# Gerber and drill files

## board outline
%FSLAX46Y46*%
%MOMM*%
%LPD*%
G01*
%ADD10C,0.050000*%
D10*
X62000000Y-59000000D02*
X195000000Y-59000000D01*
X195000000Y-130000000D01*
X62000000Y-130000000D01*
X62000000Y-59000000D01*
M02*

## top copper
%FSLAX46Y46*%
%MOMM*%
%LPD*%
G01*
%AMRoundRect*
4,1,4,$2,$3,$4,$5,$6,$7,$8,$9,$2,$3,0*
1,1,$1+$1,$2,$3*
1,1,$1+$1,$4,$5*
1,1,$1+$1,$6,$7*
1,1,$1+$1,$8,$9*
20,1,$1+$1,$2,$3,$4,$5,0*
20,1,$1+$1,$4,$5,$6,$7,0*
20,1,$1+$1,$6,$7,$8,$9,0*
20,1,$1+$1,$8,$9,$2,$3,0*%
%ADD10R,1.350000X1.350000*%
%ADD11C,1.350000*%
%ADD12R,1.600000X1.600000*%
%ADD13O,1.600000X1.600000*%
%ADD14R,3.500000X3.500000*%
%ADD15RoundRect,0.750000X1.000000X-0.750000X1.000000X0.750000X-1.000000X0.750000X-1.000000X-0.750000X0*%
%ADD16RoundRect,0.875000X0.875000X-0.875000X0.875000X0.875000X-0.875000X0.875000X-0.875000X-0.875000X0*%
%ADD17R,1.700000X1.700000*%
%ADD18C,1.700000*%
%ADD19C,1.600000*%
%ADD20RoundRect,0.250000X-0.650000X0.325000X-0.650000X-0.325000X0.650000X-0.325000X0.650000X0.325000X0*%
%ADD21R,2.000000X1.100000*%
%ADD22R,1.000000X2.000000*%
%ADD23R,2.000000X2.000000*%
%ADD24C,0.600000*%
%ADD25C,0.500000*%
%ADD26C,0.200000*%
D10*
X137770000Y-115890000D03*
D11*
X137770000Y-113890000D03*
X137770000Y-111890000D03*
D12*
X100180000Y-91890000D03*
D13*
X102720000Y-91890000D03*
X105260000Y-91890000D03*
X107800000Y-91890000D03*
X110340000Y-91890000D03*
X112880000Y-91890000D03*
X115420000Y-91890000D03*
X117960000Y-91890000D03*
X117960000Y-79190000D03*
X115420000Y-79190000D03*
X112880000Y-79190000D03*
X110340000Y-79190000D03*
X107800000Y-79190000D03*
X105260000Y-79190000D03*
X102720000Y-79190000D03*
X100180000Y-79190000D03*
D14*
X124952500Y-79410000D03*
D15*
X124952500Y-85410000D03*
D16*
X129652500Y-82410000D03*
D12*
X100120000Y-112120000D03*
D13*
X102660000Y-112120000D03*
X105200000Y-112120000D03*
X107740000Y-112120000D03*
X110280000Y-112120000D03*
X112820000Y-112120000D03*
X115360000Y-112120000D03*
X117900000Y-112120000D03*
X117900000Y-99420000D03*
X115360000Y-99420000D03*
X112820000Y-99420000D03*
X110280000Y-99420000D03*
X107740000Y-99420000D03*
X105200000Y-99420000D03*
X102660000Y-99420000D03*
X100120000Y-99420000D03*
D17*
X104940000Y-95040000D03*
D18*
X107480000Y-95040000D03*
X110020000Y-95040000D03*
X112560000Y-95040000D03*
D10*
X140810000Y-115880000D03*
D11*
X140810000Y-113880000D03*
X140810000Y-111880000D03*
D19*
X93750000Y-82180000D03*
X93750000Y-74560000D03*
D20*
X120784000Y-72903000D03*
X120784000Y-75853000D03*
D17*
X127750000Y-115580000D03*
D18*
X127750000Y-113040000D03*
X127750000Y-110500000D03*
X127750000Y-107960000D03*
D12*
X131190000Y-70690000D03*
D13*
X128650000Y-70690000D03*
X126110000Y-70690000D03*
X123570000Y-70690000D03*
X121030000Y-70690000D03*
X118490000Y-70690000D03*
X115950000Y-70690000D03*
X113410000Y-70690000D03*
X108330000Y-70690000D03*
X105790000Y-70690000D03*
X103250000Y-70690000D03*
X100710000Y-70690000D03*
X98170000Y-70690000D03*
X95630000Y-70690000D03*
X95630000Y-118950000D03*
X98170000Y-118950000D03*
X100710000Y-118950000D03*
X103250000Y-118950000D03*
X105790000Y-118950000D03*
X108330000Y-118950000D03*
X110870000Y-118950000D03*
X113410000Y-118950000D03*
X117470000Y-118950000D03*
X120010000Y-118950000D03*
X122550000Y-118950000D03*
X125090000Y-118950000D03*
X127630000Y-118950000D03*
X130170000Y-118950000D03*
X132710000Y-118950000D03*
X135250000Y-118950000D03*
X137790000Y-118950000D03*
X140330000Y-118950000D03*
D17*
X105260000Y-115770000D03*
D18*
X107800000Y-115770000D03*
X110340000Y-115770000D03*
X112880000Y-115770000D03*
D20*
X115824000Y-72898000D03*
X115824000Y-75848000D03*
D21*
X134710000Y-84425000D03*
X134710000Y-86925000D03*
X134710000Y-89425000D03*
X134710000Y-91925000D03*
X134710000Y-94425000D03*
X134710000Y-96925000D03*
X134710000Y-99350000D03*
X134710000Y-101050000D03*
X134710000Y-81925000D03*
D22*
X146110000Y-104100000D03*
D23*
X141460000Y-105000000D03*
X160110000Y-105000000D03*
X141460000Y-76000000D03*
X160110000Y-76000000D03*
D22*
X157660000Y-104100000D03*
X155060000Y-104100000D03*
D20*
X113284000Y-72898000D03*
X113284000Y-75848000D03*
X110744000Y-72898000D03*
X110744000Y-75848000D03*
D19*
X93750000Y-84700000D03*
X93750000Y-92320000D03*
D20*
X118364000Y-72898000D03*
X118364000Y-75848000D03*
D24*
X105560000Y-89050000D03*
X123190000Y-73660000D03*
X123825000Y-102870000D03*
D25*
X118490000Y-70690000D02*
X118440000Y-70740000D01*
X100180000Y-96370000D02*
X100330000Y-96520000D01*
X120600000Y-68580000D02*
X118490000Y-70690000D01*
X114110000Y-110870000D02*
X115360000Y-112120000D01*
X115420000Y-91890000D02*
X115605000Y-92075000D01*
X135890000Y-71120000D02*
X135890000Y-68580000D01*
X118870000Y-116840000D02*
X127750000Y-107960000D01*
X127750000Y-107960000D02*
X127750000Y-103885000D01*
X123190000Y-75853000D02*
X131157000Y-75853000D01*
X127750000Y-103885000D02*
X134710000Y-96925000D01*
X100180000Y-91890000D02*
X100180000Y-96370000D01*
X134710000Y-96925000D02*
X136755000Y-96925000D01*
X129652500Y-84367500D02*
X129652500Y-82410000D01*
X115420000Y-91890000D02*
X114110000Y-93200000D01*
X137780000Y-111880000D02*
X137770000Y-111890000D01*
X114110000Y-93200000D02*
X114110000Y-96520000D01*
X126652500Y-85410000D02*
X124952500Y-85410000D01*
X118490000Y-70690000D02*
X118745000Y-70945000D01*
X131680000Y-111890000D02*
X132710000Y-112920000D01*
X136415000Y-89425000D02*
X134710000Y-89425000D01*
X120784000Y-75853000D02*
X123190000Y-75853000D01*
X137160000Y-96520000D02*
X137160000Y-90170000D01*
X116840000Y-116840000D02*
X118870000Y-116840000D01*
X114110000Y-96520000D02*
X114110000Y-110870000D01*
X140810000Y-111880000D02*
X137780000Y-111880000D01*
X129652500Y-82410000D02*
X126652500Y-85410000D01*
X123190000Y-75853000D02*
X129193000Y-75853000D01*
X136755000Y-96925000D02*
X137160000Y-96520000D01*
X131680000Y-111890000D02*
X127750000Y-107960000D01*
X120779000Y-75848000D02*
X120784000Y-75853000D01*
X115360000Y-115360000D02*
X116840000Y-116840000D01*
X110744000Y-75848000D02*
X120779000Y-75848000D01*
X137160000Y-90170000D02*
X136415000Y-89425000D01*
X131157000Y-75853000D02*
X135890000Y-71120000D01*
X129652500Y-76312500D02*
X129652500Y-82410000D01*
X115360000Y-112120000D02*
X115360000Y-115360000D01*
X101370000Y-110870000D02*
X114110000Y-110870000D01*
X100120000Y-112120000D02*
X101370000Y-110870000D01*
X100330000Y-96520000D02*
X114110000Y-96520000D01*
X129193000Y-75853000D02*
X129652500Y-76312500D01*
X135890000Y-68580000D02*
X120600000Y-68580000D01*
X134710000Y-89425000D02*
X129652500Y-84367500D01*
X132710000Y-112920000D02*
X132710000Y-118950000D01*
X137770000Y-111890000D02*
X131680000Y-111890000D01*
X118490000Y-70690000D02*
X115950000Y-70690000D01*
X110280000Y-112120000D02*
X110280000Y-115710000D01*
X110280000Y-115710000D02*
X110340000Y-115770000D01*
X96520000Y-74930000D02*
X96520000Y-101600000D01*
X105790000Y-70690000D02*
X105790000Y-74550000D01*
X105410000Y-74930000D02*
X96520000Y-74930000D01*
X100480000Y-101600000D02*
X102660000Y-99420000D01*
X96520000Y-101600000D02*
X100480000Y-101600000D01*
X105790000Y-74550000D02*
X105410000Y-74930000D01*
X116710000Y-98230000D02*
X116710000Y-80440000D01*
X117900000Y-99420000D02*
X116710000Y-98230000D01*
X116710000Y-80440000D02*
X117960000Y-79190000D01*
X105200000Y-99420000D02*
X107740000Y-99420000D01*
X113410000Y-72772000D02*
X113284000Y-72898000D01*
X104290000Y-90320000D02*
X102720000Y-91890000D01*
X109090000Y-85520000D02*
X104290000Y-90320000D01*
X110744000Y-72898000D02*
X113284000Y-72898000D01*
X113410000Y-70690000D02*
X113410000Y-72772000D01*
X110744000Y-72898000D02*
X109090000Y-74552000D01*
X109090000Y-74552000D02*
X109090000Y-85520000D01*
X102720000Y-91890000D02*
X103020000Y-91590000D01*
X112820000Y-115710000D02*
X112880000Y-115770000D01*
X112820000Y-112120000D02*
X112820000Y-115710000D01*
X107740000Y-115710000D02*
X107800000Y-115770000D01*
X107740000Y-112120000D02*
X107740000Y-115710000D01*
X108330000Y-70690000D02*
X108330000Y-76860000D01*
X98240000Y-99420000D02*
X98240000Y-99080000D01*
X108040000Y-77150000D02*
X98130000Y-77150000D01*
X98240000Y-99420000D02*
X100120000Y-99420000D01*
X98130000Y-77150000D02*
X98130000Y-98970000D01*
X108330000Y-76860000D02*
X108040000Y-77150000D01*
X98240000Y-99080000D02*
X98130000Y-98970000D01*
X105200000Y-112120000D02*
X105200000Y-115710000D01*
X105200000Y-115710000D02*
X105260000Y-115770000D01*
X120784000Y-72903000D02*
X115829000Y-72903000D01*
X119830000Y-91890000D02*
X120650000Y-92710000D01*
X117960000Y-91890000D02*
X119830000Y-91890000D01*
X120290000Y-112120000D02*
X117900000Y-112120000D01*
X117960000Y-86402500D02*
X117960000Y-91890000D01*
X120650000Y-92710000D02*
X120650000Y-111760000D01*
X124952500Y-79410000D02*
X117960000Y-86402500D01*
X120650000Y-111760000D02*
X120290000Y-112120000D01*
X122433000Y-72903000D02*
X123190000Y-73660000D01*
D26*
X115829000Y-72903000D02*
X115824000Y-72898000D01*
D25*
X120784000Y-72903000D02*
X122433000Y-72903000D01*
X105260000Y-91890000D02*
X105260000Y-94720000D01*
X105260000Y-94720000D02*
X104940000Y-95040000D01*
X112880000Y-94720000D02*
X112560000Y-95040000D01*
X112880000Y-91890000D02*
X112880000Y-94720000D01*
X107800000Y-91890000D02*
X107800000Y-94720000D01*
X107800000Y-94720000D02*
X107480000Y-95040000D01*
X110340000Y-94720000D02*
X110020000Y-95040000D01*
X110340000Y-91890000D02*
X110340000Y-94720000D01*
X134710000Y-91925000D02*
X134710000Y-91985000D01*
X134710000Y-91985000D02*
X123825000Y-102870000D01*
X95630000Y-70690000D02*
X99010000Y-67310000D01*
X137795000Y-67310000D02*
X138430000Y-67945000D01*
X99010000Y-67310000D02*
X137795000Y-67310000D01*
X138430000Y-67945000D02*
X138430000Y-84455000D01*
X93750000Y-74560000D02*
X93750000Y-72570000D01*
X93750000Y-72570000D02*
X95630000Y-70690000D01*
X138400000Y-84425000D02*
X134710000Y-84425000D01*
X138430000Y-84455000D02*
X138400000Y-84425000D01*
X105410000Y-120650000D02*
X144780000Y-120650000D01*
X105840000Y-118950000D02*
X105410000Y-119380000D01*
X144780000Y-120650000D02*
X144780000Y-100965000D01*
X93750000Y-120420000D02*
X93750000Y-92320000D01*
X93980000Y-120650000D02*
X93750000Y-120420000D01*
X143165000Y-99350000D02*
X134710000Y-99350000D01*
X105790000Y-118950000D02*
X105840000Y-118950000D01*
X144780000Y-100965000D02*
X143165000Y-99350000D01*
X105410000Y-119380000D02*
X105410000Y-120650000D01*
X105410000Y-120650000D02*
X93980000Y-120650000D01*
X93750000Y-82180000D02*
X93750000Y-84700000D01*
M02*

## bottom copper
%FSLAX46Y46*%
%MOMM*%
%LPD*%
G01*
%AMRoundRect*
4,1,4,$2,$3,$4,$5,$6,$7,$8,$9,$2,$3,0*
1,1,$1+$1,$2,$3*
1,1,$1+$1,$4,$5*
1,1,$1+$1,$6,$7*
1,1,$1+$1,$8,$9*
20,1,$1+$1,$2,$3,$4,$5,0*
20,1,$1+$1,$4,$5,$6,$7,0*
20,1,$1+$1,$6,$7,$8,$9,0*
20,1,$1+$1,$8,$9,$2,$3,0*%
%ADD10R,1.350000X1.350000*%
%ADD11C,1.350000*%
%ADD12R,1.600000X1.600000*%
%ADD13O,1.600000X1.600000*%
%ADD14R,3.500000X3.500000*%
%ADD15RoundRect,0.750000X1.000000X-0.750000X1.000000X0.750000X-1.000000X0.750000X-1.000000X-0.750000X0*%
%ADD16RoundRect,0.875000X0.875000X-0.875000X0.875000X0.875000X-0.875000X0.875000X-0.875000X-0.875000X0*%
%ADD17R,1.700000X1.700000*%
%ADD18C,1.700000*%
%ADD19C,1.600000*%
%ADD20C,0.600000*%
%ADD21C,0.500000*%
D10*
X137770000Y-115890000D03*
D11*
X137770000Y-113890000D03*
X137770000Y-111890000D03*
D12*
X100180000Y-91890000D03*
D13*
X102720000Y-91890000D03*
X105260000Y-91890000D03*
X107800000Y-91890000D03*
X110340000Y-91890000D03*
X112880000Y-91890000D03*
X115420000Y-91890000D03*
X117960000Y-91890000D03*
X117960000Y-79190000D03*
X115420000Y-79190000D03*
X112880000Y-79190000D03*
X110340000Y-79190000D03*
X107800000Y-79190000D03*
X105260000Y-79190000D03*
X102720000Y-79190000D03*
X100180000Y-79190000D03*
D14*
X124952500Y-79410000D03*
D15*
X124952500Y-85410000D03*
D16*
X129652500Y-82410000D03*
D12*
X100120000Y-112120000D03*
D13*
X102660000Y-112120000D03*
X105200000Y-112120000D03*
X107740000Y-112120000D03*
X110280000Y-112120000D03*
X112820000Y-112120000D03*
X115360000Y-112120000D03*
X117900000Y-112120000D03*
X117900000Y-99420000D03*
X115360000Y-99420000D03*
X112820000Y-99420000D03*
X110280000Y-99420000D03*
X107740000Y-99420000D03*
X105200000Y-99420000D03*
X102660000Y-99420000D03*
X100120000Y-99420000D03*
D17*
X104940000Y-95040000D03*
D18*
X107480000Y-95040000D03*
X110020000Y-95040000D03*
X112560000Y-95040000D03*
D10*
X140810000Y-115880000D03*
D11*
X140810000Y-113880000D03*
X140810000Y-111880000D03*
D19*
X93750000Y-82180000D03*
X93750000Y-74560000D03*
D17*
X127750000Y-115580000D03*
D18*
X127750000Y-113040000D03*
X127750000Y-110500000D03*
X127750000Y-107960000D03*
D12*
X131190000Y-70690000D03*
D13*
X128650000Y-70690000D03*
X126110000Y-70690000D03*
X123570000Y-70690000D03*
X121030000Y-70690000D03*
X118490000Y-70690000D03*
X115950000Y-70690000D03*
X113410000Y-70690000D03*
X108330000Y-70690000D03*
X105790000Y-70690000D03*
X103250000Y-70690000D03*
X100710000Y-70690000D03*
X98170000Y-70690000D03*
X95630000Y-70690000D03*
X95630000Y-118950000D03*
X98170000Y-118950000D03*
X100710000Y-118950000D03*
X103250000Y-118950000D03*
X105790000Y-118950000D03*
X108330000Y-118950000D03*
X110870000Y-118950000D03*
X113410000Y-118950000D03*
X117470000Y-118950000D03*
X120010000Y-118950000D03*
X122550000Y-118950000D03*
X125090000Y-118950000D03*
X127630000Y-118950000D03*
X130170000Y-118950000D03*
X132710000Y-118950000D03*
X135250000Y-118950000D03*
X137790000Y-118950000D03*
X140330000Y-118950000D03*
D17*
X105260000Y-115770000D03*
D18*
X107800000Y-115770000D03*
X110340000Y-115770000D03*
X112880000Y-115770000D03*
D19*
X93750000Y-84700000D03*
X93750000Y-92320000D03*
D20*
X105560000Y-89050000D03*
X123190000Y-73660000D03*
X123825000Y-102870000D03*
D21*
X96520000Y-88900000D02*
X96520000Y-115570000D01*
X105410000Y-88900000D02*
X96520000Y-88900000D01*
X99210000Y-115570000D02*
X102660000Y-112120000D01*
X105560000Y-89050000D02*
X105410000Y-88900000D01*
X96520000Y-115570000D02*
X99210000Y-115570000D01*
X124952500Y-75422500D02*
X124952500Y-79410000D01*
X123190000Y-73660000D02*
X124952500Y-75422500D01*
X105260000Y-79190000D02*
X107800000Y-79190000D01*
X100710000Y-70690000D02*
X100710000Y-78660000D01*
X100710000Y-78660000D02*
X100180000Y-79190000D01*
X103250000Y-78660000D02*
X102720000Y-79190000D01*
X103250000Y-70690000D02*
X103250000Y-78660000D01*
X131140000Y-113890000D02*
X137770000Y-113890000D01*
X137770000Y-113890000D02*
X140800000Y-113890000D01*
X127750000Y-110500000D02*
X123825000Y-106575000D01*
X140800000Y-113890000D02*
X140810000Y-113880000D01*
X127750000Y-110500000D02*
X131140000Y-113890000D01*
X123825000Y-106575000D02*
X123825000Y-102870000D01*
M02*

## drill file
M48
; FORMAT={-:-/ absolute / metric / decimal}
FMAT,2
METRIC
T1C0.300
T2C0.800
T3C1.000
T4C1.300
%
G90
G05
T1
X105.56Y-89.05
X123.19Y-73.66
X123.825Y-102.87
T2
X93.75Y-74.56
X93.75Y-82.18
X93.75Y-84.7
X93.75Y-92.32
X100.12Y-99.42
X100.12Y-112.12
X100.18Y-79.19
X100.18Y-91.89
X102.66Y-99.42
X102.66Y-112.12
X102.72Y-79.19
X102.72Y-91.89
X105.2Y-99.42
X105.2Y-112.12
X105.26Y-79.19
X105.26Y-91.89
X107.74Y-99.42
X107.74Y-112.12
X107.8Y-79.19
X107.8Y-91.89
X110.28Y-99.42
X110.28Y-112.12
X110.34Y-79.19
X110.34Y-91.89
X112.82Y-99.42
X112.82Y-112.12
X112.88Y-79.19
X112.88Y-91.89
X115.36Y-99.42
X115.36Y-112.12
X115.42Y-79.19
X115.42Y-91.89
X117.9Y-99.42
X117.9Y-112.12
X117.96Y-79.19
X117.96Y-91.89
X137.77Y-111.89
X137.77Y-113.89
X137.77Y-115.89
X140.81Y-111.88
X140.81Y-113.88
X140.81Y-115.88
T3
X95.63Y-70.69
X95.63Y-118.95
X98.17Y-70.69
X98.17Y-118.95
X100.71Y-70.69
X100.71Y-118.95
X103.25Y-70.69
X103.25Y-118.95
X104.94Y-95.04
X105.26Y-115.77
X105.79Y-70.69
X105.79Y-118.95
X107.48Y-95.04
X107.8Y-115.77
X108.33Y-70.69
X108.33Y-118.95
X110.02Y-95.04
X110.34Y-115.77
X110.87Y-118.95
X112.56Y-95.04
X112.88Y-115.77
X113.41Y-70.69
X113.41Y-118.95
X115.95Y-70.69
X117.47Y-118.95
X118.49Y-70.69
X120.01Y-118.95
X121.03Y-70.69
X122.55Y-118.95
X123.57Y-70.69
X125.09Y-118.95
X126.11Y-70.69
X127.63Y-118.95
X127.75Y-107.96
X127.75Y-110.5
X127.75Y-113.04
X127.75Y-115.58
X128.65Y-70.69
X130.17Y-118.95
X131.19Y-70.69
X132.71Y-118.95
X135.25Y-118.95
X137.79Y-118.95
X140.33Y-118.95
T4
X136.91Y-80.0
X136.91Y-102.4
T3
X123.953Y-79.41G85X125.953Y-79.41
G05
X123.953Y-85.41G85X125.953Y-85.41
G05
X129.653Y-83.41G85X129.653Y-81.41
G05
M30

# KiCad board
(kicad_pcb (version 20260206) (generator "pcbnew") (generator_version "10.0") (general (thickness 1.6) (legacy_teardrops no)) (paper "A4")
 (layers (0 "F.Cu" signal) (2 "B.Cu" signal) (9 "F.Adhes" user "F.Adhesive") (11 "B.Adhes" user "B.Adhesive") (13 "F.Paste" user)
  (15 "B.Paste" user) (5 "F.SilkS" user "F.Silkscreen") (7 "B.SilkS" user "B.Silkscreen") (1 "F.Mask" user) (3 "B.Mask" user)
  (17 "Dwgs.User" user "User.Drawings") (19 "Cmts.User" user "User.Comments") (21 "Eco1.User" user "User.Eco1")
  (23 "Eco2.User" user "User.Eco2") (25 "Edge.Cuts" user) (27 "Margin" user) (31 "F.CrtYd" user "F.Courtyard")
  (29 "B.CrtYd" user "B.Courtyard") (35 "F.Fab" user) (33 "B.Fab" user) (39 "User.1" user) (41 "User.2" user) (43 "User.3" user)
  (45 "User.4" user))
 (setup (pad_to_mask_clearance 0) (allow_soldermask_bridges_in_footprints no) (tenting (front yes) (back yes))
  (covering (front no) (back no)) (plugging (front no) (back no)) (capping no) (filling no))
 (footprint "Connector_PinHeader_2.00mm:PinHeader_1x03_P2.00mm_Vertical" (layer "F.Cu") (at 137.77 115.89 180)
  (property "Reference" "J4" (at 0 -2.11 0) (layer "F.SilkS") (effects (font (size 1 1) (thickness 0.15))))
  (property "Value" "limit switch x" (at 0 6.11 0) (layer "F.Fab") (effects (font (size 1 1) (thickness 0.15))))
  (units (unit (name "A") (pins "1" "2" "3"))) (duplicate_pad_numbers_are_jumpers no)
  (pad "1" thru_hole rect (at 0 0 180) (size 1.35 1.35) (drill 0.8) (layers "*.Cu" "*.Mask") (remove_unused_layers no) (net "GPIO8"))
  (pad "2" thru_hole circle (at 0 2 180) (size 1.35 1.35) (drill 0.8) (layers "*.Cu" "*.Mask") (remove_unused_layers no) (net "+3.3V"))
  (pad "3" thru_hole circle (at 0 4 180) (size 1.35 1.35) (drill 0.8) (layers "*.Cu" "*.Mask") (remove_unused_layers no) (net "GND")))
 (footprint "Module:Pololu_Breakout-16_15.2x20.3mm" (layer "F.Cu") (at 100.18 91.89 90)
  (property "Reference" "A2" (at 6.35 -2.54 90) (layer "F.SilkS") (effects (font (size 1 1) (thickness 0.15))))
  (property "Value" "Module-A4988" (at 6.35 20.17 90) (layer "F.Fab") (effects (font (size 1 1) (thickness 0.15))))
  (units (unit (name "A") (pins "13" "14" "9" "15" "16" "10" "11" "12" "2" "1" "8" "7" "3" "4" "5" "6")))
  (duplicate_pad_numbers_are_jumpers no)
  (pad "1" thru_hole rect (at 0 0 90) (size 1.6 1.6) (drill 0.8) (layers "*.Cu" "*.Mask") (remove_unused_layers no) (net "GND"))
  (pad "2" thru_hole oval (at 0 2.54 90) (size 1.6 1.6) (drill 0.8) (layers "*.Cu" "*.Mask") (remove_unused_layers no) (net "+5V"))
  (pad "3" thru_hole oval (at 0 5.08 90) (size 1.6 1.6) (drill 0.8) (layers "*.Cu" "*.Mask") (remove_unused_layers no) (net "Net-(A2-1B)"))
  (pad "4" thru_hole oval (at 0 7.62 90) (size 1.6 1.6) (drill 0.8) (layers "*.Cu" "*.Mask") (remove_unused_layers no) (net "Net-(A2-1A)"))
  (pad "5" thru_hole oval (at 0 10.16 90) (size 1.6 1.6) (drill 0.8) (layers "*.Cu" "*.Mask") (remove_unused_layers no) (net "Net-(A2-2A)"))
  (pad "6" thru_hole oval (at 0 12.7 90) (size 1.6 1.6) (drill 0.8) (layers "*.Cu" "*.Mask") (remove_unused_layers no) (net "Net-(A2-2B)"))
  (pad "7" thru_hole oval (at 0 15.24 90) (size 1.6 1.6) (drill 0.8) (layers "*.Cu" "*.Mask") (remove_unused_layers no) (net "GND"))
  (pad "8" thru_hole oval (at 0 17.78 90) (size 1.6 1.6) (drill 0.8) (layers "*.Cu" "*.Mask") (remove_unused_layers no) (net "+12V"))
  (pad "9" thru_hole oval (at 12.7 17.78 90) (size 1.6 1.6) (drill 0.8) (layers "*.Cu" "*.Mask") (remove_unused_layers no) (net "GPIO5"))
  (pad "10" thru_hole oval (at 12.7 15.24 90) (size 1.6 1.6) (drill 0.8) (layers "*.Cu" "*.Mask") (remove_unused_layers no)
   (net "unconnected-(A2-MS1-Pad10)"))
  (pad "11" thru_hole oval (at 12.7 12.7 90) (size 1.6 1.6) (drill 0.8) (layers "*.Cu" "*.Mask") (remove_unused_layers no)
   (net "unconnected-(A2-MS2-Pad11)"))
  (pad "12" thru_hole oval (at 12.7 10.16 90) (size 1.6 1.6) (drill 0.8) (layers "*.Cu" "*.Mask") (remove_unused_layers no)
   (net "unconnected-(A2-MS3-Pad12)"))
  (pad "13" thru_hole oval (at 12.7 7.62 90) (size 1.6 1.6) (drill 0.8) (layers "*.Cu" "*.Mask") (remove_unused_layers no)
   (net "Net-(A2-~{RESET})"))
  (pad "14" thru_hole oval (at 12.7 5.08 90) (size 1.6 1.6) (drill 0.8) (layers "*.Cu" "*.Mask") (remove_unused_layers no)
   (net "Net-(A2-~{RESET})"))
  (pad "15" thru_hole oval (at 12.7 2.54 90) (size 1.6 1.6) (drill 0.8) (layers "*.Cu" "*.Mask") (remove_unused_layers no) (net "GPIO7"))
  (pad "16" thru_hole oval (at 12.7 0 90) (size 1.6 1.6) (drill 0.8) (layers "*.Cu" "*.Mask") (remove_unused_layers no) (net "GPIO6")))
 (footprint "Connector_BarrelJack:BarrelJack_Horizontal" (layer "F.Cu") (at 124.9525 79.41 90)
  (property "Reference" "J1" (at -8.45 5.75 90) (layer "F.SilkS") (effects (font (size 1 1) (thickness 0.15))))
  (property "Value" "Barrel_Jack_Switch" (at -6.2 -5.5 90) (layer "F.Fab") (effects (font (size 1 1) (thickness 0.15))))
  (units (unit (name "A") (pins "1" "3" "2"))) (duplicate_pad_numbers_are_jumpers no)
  (pad "1" thru_hole rect (at 0 0 90) (size 3.5 3.5) (drill oval 1 3) (layers "*.Cu" "*.Mask") (remove_unused_layers no) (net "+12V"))
  (pad "2" thru_hole roundrect (at -6 0 90) (size 3 3.5) (drill oval 1 3) (layers "*.Cu" "*.Mask") (remove_unused_layers no)
   (roundrect_rratio 0.25) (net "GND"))
  (pad "3" thru_hole roundrect (at -3 4.7 90) (size 3.5 3.5) (drill oval 3 1) (layers "*.Cu" "*.Mask") (remove_unused_layers no)
   (roundrect_rratio 0.25) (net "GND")))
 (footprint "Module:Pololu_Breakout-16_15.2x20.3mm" (layer "F.Cu") (at 100.12 112.12 90)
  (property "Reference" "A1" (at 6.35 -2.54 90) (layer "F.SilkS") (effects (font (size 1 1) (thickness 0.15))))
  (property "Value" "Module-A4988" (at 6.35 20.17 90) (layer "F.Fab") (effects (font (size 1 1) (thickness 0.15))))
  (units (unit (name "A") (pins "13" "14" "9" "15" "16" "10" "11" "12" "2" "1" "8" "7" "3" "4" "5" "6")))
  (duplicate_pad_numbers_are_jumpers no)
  (pad "1" thru_hole rect (at 0 0 90) (size 1.6 1.6) (drill 0.8) (layers "*.Cu" "*.Mask") (remove_unused_layers no) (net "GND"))
  (pad "2" thru_hole oval (at 0 2.54 90) (size 1.6 1.6) (drill 0.8) (layers "*.Cu" "*.Mask") (remove_unused_layers no) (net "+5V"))
  (pad "3" thru_hole oval (at 0 5.08 90) (size 1.6 1.6) (drill 0.8) (layers "*.Cu" "*.Mask") (remove_unused_layers no) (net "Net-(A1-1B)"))
  (pad "4" thru_hole oval (at 0 7.62 90) (size 1.6 1.6) (drill 0.8) (layers "*.Cu" "*.Mask") (remove_unused_layers no) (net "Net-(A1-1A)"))
  (pad "5" thru_hole oval (at 0 10.16 90) (size 1.6 1.6) (drill 0.8) (layers "*.Cu" "*.Mask") (remove_unused_layers no) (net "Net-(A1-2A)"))
  (pad "6" thru_hole oval (at 0 12.7 90) (size 1.6 1.6) (drill 0.8) (layers "*.Cu" "*.Mask") (remove_unused_layers no) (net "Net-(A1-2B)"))
  (pad "7" thru_hole oval (at 0 15.24 90) (size 1.6 1.6) (drill 0.8) (layers "*.Cu" "*.Mask") (remove_unused_layers no) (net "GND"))
  (pad "8" thru_hole oval (at 0 17.78 90) (size 1.6 1.6) (drill 0.8) (layers "*.Cu" "*.Mask") (remove_unused_layers no) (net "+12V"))
  (pad "9" thru_hole oval (at 12.7 17.78 90) (size 1.6 1.6) (drill 0.8) (layers "*.Cu" "*.Mask") (remove_unused_layers no) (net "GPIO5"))
  (pad "10" thru_hole oval (at 12.7 15.24 90) (size 1.6 1.6) (drill 0.8) (layers "*.Cu" "*.Mask") (remove_unused_layers no)
   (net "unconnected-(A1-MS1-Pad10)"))
  (pad "11" thru_hole oval (at 12.7 12.7 90) (size 1.6 1.6) (drill 0.8) (layers "*.Cu" "*.Mask") (remove_unused_layers no)
   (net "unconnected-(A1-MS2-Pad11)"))
  (pad "12" thru_hole oval (at 12.7 10.16 90) (size 1.6 1.6) (drill 0.8) (layers "*.Cu" "*.Mask") (remove_unused_layers no)
   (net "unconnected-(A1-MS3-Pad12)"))
  (pad "13" thru_hole oval (at 12.7 7.62 90) (size 1.6 1.6) (drill 0.8) (layers "*.Cu" "*.Mask") (remove_unused_layers no)
   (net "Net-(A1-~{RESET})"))
  (pad "14" thru_hole oval (at 12.7 5.08 90) (size 1.6 1.6) (drill 0.8) (layers "*.Cu" "*.Mask") (remove_unused_layers no)
   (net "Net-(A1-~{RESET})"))
  (pad "15" thru_hole oval (at 12.7 2.54 90) (size 1.6 1.6) (drill 0.8) (layers "*.Cu" "*.Mask") (remove_unused_layers no) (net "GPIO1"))
  (pad "16" thru_hole oval (at 12.7 0 90) (size 1.6 1.6) (drill 0.8) (layers "*.Cu" "*.Mask") (remove_unused_layers no) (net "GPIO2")))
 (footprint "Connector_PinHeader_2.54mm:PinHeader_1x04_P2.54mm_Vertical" (layer "F.Cu") (at 104.94 95.04 90)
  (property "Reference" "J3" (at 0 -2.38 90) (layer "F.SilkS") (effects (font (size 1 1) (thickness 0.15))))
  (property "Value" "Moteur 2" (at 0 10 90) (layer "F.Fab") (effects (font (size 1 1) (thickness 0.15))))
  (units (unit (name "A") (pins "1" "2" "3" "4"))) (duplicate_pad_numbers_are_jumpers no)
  (pad "1" thru_hole rect (at 0 0 90) (size 1.7 1.7) (drill 1) (layers "*.Cu" "*.Mask") (remove_unused_layers no) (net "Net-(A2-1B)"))
  (pad "2" thru_hole circle (at 0 2.54 90) (size 1.7 1.7) (drill 1) (layers "*.Cu" "*.Mask") (remove_unused_layers no) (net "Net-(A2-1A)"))
  (pad "3" thru_hole circle (at 0 5.08 90) (size 1.7 1.7) (drill 1) (layers "*.Cu" "*.Mask") (remove_unused_layers no) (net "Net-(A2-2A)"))
  (pad "4" thru_hole circle (at 0 7.62 90) (size 1.7 1.7) (drill 1) (layers "*.Cu" "*.Mask") (remove_unused_layers no) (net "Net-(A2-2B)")))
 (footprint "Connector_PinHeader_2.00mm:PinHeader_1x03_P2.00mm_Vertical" (layer "F.Cu") (at 140.81 115.88 180)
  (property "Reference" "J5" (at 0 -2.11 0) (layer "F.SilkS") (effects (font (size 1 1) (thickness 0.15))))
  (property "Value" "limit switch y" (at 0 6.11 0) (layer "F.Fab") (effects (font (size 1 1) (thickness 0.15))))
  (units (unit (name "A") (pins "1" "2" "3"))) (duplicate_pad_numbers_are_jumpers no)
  (pad "1" thru_hole rect (at 0 0 180) (size 1.35 1.35) (drill 0.8) (layers "*.Cu" "*.Mask") (remove_unused_layers no) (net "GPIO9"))
  (pad "2" thru_hole circle (at 0 2 180) (size 1.35 1.35) (drill 0.8) (layers "*.Cu" "*.Mask") (remove_unused_layers no) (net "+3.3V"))
  (pad "3" thru_hole circle (at 0 4 180) (size 1.35 1.35) (drill 0.8) (layers "*.Cu" "*.Mask") (remove_unused_layers no) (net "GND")))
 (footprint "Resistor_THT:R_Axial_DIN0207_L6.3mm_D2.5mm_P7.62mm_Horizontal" (layer "F.Cu") (at 93.75 82.18 90)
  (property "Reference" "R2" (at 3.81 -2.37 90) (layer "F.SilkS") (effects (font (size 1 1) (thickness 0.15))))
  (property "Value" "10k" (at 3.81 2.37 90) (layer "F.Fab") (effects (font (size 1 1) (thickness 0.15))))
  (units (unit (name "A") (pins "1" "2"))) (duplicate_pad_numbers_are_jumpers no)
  (pad "1" thru_hole circle (at 0 0 90) (size 1.6 1.6) (drill 0.8) (layers "*.Cu" "*.Mask") (remove_unused_layers no) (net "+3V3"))
  (pad "2" thru_hole circle (at 7.62 0 90) (size 1.6 1.6) (drill 0.8) (layers "*.Cu" "*.Mask") (remove_unused_layers no) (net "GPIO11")))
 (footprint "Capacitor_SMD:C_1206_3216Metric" (layer "F.Cu") (at 120.784 74.378 -90)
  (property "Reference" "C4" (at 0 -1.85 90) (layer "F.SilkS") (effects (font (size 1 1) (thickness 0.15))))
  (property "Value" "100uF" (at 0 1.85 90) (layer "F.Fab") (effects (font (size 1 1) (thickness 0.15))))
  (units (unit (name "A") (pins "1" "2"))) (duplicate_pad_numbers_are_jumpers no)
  (pad "1" smd roundrect (at -1.475 0 270) (size 1.15 1.8) (layers "F.Cu" "F.Mask" "F.Paste") (roundrect_rratio 0.217391) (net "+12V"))
  (pad "2" smd roundrect (at 1.475 0 270) (size 1.15 1.8) (layers "F.Cu" "F.Mask" "F.Paste") (roundrect_rratio 0.217391) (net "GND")))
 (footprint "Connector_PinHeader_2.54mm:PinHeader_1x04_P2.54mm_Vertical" (layer "F.Cu") (at 127.75 115.58 180)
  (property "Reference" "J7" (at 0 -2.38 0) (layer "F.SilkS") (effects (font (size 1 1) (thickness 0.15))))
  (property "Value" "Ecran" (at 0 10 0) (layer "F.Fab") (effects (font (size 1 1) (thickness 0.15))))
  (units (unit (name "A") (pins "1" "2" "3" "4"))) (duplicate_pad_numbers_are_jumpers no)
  (pad "1" thru_hole rect (at 0 0 180) (size 1.7 1.7) (drill 1) (layers "*.Cu" "*.Mask") (remove_unused_layers no) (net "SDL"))
  (pad "2" thru_hole circle (at 0 2.54 180) (size 1.7 1.7) (drill 1) (layers "*.Cu" "*.Mask") (remove_unused_layers no) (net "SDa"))
  (pad "3" thru_hole circle (at 0 5.08 180) (size 1.7 1.7) (drill 1) (layers "*.Cu" "*.Mask") (remove_unused_layers no) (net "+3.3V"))
  (pad "4" thru_hole circle (at 0 7.62 180) (size 1.7 1.7) (drill 1) (layers "*.Cu" "*.Mask") (remove_unused_layers no) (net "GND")))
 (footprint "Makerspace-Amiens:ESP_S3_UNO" (layer "F.Cu") (at 131.19 70.69)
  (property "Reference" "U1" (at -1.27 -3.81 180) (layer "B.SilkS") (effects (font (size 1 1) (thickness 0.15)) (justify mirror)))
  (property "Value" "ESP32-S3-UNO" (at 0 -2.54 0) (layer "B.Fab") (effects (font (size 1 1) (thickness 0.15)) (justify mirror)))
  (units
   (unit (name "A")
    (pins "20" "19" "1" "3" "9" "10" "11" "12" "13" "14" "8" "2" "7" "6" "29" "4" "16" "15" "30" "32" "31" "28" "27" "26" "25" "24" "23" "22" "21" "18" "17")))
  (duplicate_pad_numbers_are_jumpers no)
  (pad "1" thru_hole rect (at 0 0 270) (size 1.6 1.6) (drill 1) (layers "*.Cu" "*.Mask") (remove_unused_layers no)
   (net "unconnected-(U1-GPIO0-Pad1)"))
  (pad "2" thru_hole oval (at -2.54 0 270) (size 1.6 1.6) (drill 1) (layers "*.Cu" "*.Mask") (remove_unused_layers no)
   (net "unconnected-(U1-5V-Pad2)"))
  (pad "3" thru_hole oval (at -5.08 0 270) (size 1.6 1.6) (drill 1) (layers "*.Cu" "*.Mask") (remove_unused_layers no)
   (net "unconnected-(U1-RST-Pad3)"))
  (pad "4" thru_hole oval (at -7.62 0 270) (size 1.6 1.6) (drill 1) (layers "*.Cu" "*.Mask") (remove_unused_layers no)
   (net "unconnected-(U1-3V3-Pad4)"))
  (pad "5" thru_hole oval (at -10.16 0 270) (size 1.6 1.6) (drill 1) (layers "*.Cu" "*.Mask") (remove_unused_layers no))
  (pad "6" thru_hole oval (at -12.7 0 270) (size 1.6 1.6) (drill 1) (layers "*.Cu" "*.Mask") (remove_unused_layers no) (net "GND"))
  (pad "7" thru_hole oval (at -15.24 0 270) (size 1.6 1.6) (drill 1) (layers "*.Cu" "*.Mask") (remove_unused_layers no) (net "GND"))
  (pad "8" thru_hole oval (at -17.78 0 270) (size 1.6 1.6) (drill 1) (layers "*.Cu" "*.Mask") (remove_unused_layers no) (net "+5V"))
  (pad "9" thru_hole oval (at -22.86 0 270) (size 1.6 1.6) (drill 1) (layers "*.Cu" "*.Mask") (remove_unused_layers no) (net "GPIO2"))
  (pad "10" thru_hole oval (at -25.4 0 270) (size 1.6 1.6) (drill 1) (layers "*.Cu" "*.Mask") (remove_unused_layers no) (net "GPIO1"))
  (pad "11" thru_hole oval (at -27.94 0 270) (size 1.6 1.6) (drill 1) (layers "*.Cu" "*.Mask") (remove_unused_layers no) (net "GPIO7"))
  (pad "12" thru_hole oval (at -30.48 0 270) (size 1.6 1.6) (drill 1) (layers "*.Cu" "*.Mask") (remove_unused_layers no) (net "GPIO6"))
  (pad "13" thru_hole oval (at -33.02 0 270) (size 1.6 1.6) (drill 1) (layers "*.Cu" "*.Mask") (remove_unused_layers no) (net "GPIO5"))
  (pad "14" thru_hole oval (at -35.56 0 270) (size 1.6 1.6) (drill 1) (layers "*.Cu" "*.Mask") (remove_unused_layers no) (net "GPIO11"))
  (pad "15" thru_hole oval (at -35.56 48.26 270) (size 1.6 1.6) (drill 1) (layers "*.Cu" "*.Mask") (remove_unused_layers no)
   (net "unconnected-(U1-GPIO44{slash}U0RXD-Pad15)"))
  (pad "16" thru_hole oval (at -33.02 48.26 270) (size 1.6 1.6) (drill 1) (layers "*.Cu" "*.Mask") (remove_unused_layers no)
   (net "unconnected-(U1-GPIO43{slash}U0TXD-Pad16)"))
  (pad "17" thru_hole oval (at -30.48 48.26 270) (size 1.6 1.6) (drill 1) (layers "*.Cu" "*.Mask") (remove_unused_layers no) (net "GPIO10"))
  (pad "18" thru_hole oval (at -27.94 48.26 270) (size 1.6 1.6) (drill 1) (layers "*.Cu" "*.Mask") (remove_unused_layers no)
   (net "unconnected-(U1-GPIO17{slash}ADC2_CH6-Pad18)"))
  (pad "19" thru_hole oval (at -25.4 48.26 270) (size 1.6 1.6) (drill 1) (layers "*.Cu" "*.Mask") (remove_unused_layers no) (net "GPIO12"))
  (pad "20" thru_hole oval (at -22.86 48.26 270) (size 1.6 1.6) (drill 1) (layers "*.Cu" "*.Mask") (remove_unused_layers no)
   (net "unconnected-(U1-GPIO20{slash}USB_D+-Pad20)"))
  (pad "21" thru_hole oval (at -20.32 48.26 270) (size 1.6 1.6) (drill 1) (layers "*.Cu" "*.Mask") (remove_unused_layers no)
   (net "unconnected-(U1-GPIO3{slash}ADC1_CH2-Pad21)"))
  (pad "22" thru_hole oval (at -17.78 48.26 270) (size 1.6 1.6) (drill 1) (layers "*.Cu" "*.Mask") (remove_unused_layers no)
   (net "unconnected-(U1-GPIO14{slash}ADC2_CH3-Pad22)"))
  (pad "23" thru_hole oval (at -13.72 48.26 270) (size 1.6 1.6) (drill 1) (layers "*.Cu" "*.Mask") (remove_unused_layers no)
   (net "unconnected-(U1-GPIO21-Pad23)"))
  (pad "24" thru_hole oval (at -11.18 48.26 270) (size 1.6 1.6) (drill 1) (layers "*.Cu" "*.Mask") (remove_unused_layers no)
   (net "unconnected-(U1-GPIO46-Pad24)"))
  (pad "25" thru_hole oval (at -8.64 48.26 270) (size 1.6 1.6) (drill 1) (layers "*.Cu" "*.Mask") (remove_unused_layers no)
   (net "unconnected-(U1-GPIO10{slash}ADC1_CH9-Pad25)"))
  (pad "26" thru_hole oval (at -6.1 48.26 270) (size 1.6 1.6) (drill 1) (layers "*.Cu" "*.Mask") (remove_unused_layers no) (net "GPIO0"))
  (pad "27" thru_hole oval (at -3.56 48.26 270) (size 1.6 1.6) (drill 1) (layers "*.Cu" "*.Mask") (remove_unused_layers no) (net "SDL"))
  (pad "28" thru_hole oval (at -1.02 48.26 270) (size 1.6 1.6) (drill 1) (layers "*.Cu" "*.Mask") (remove_unused_layers no) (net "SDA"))
  (pad "29" thru_hole oval (at 1.52 48.26 270) (size 1.6 1.6) (drill 1) (layers "*.Cu" "*.Mask") (remove_unused_layers no) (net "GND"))
  (pad "30" thru_hole oval (at 4.06 48.26 270) (size 1.6 1.6) (drill 1) (layers "*.Cu" "*.Mask") (remove_unused_layers no)
   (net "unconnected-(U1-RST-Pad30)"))
  (pad "31" thru_hole oval (at 6.6 48.26 270) (size 1.6 1.6) (drill 1) (layers "*.Cu" "*.Mask") (remove_unused_layers no) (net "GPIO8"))
  (pad "32" thru_hole oval (at 9.14 48.26 270) (size 1.6 1.6) (drill 1) (layers "*.Cu" "*.Mask") (remove_unused_layers no) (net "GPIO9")))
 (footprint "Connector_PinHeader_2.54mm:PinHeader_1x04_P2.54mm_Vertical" (layer "F.Cu") (at 105.26 115.77 90)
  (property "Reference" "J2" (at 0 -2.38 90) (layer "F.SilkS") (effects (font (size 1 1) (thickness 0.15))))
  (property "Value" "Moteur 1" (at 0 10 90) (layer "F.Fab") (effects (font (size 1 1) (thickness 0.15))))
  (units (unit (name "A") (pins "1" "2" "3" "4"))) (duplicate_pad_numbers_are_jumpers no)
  (pad "1" thru_hole rect (at 0 0 90) (size 1.7 1.7) (drill 1) (layers "*.Cu" "*.Mask") (remove_unused_layers no) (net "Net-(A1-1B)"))
  (pad "2" thru_hole circle (at 0 2.54 90) (size 1.7 1.7) (drill 1) (layers "*.Cu" "*.Mask") (remove_unused_layers no) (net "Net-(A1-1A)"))
  (pad "3" thru_hole circle (at 0 5.08 90) (size 1.7 1.7) (drill 1) (layers "*.Cu" "*.Mask") (remove_unused_layers no) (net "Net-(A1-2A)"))
  (pad "4" thru_hole circle (at 0 7.62 90) (size 1.7 1.7) (drill 1) (layers "*.Cu" "*.Mask") (remove_unused_layers no) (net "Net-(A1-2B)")))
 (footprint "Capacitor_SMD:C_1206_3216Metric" (layer "F.Cu") (at 115.824 74.373 -90)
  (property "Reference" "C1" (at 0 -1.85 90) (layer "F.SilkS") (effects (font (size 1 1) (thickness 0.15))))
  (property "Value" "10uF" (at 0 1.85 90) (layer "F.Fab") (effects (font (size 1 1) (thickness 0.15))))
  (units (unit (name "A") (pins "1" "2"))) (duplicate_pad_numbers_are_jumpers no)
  (pad "1" smd roundrect (at -1.475 0 270) (size 1.15 1.8) (layers "F.Cu" "F.Mask" "F.Paste") (roundrect_rratio 0.217391) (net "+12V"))
  (pad "2" smd roundrect (at 1.475 0 270) (size 1.15 1.8) (layers "F.Cu" "F.Mask" "F.Paste") (roundrect_rratio 0.217391) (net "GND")))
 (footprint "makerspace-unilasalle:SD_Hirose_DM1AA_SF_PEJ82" (layer "F.Cu") (at 149.66 90.5 90)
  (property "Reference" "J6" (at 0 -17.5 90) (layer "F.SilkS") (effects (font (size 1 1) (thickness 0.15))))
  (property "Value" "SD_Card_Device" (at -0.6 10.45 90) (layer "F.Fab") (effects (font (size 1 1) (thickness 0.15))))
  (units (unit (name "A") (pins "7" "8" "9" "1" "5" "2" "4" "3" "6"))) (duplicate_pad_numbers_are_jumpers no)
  (pad "" np_thru_hole circle (at -11.9 -12.75 90) (size 1.3 1.3) (drill 1.3) (layers "*.Cu" "*.Mask"))
  (pad "" np_thru_hole circle (at 10.5 -12.75 90) (size 1.3 1.3) (drill 1.3) (layers "*.Cu" "*.Mask"))
  (pad "1" smd rect (at 6.075 -14.95 90) (size 1.1 2) (layers "F.Cu" "F.Mask" "F.Paste") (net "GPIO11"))
  (pad "2" smd rect (at 3.575 -14.95 90) (size 1.1 2) (layers "F.Cu" "F.Mask" "F.Paste") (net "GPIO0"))
  (pad "3" smd rect (at 1.075 -14.95 90) (size 1.1 2) (layers "F.Cu" "F.Mask" "F.Paste") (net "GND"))
  (pad "4" smd rect (at -1.425 -14.95 90) (size 1.1 2) (layers "F.Cu" "F.Mask" "F.Paste") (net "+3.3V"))
  (pad "5" smd rect (at -3.925 -14.95 90) (size 1.1 2) (layers "F.Cu" "F.Mask" "F.Paste") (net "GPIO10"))
  (pad "6" smd rect (at -6.425 -14.95 90) (size 1.1 2) (layers "F.Cu" "F.Mask" "F.Paste") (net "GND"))
  (pad "7" smd rect (at -8.85 -14.95 90) (size 1.1 2) (layers "F.Cu" "F.Mask" "F.Paste") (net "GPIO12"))
  (pad "8" smd rect (at -10.55 -14.95 90) (size 1.1 2) (layers "F.Cu" "F.Mask" "F.Paste") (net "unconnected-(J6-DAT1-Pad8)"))
  (pad "9" smd rect (at 8.575 -14.95 90) (size 1.1 2) (layers "F.Cu" "F.Mask" "F.Paste") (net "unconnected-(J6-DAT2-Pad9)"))
  (pad "CP" smd rect (at -13.6 -3.55 90) (size 2 1) (layers "F.Cu" "F.Mask" "F.Paste"))
  (pad "SH" smd rect (at -14.5 -8.2 90) (size 2 2) (layers "F.Cu" "F.Mask" "F.Paste"))
  (pad "SH" smd rect (at -14.5 10.45 90) (size 2 2) (layers "F.Cu" "F.Mask" "F.Paste"))
  (pad "SH" smd rect (at 14.5 -8.2 90) (size 2 2) (layers "F.Cu" "F.Mask" "F.Paste"))
  (pad "SH" smd rect (at 14.5 10.45 90) (size 2 2) (layers "F.Cu" "F.Mask" "F.Paste"))
  (pad "SW" smd rect (at -13.6 8 90) (size 2 1) (layers "F.Cu" "F.Mask" "F.Paste"))
  (pad "WP" smd rect (at -13.6 5.4 90) (size 2 1) (layers "F.Cu" "F.Mask" "F.Paste")))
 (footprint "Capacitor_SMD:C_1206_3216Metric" (layer "F.Cu") (at 113.284 74.373 -90)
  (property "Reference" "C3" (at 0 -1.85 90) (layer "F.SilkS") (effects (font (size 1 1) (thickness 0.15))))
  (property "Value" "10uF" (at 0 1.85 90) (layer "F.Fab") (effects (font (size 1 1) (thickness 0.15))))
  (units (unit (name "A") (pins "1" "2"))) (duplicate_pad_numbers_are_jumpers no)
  (pad "1" smd roundrect (at -1.475 0 270) (size 1.15 1.8) (layers "F.Cu" "F.Mask" "F.Paste") (roundrect_rratio 0.217391) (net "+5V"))
  (pad "2" smd roundrect (at 1.475 0 270) (size 1.15 1.8) (layers "F.Cu" "F.Mask" "F.Paste") (roundrect_rratio 0.217391) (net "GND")))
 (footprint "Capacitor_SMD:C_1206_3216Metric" (layer "F.Cu") (at 110.744 74.373 -90)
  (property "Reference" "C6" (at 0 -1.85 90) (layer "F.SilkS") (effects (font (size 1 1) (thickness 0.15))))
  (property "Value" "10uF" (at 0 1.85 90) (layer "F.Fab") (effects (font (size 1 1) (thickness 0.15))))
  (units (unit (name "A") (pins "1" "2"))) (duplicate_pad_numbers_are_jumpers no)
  (pad "1" smd roundrect (at -1.475 0 270) (size 1.15 1.8) (layers "F.Cu" "F.Mask" "F.Paste") (roundrect_rratio 0.217391) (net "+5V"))
  (pad "2" smd roundrect (at 1.475 0 270) (size 1.15 1.8) (layers "F.Cu" "F.Mask" "F.Paste") (roundrect_rratio 0.217391) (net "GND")))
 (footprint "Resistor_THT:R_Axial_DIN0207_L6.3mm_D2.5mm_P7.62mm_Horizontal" (layer "F.Cu") (at 93.75 84.7 -90)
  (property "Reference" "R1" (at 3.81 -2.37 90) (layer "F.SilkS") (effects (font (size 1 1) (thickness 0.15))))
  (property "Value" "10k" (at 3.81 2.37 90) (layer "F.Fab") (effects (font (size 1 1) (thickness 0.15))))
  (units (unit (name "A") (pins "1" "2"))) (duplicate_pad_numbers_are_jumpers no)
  (pad "1" thru_hole circle (at 0 0 270) (size 1.6 1.6) (drill 0.8) (layers "*.Cu" "*.Mask") (remove_unused_layers no) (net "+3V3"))
  (pad "2" thru_hole circle (at 7.62 0 270) (size 1.6 1.6) (drill 0.8) (layers "*.Cu" "*.Mask") (remove_unused_layers no) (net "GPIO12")))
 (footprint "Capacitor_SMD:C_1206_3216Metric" (layer "F.Cu") (at 118.364 74.373 -90)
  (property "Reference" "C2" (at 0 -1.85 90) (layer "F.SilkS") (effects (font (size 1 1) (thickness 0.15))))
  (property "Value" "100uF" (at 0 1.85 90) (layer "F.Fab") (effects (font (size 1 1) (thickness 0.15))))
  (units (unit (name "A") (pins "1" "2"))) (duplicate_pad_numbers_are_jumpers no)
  (pad "1" smd roundrect (at -1.475 0 270) (size 1.15 1.8) (layers "F.Cu" "F.Mask" "F.Paste") (roundrect_rratio 0.217391) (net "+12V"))
  (pad "2" smd roundrect (at 1.475 0 270) (size 1.15 1.8) (layers "F.Cu" "F.Mask" "F.Paste") (roundrect_rratio 0.217391) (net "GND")))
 (gr_rect (start 62 59) (end 195 130) (stroke (width 0.05) (type default)) (fill no) (layer "Edge.Cuts"))
 (segment (start 118.49 70.69) (end 118.44 70.74) (width 0.5) (layer "F.Cu") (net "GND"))
 (segment (start 100.18 96.37) (end 100.33 96.52) (width 0.5) (layer "F.Cu") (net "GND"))
 (segment (start 120.6 68.58) (end 118.49 70.69) (width 0.5) (layer "F.Cu") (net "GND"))
 (segment (start 114.11 110.87) (end 115.36 112.12) (width 0.5) (layer "F.Cu") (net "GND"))
 (segment (start 115.42 91.89) (end 115.605 92.075) (width 0.5) (layer "F.Cu") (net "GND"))
 (segment (start 135.89 71.12) (end 135.89 68.58) (width 0.5) (layer "F.Cu") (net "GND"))
 (segment (start 118.87 116.84) (end 127.75 107.96) (width 0.5) (layer "F.Cu") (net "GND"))
 (segment (start 127.75 107.96) (end 127.75 103.885) (width 0.5) (layer "F.Cu") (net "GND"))
 (segment (start 123.19 75.853) (end 131.157 75.853) (width 0.5) (layer "F.Cu") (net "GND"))
 (segment (start 127.75 103.885) (end 134.71 96.925) (width 0.5) (layer "F.Cu") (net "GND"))
 (segment (start 100.18 91.89) (end 100.18 96.37) (width 0.5) (layer "F.Cu") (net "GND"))
 (segment (start 134.71 96.925) (end 136.755 96.925) (width 0.5) (layer "F.Cu") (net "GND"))
 (segment (start 129.6525 84.3675) (end 129.6525 82.41) (width 0.5) (layer "F.Cu") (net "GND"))
 (segment (start 115.42 91.89) (end 114.11 93.2) (width 0.5) (layer "F.Cu") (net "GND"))
 (segment (start 137.78 111.88) (end 137.77 111.89) (width 0.5) (layer "F.Cu") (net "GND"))
 (segment (start 114.11 93.2) (end 114.11 96.52) (width 0.5) (layer "F.Cu") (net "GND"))
 (segment (start 126.6525 85.41) (end 124.9525 85.41) (width 0.5) (layer "F.Cu") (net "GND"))
 (segment (start 118.49 70.69) (end 118.745 70.945) (width 0.5) (layer "F.Cu") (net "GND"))
 (segment (start 131.68 111.89) (end 132.71 112.92) (width 0.5) (layer "F.Cu") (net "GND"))
 (segment (start 136.415 89.425) (end 134.71 89.425) (width 0.5) (layer "F.Cu") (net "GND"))
 (segment (start 120.784 75.853) (end 123.19 75.853) (width 0.5) (layer "F.Cu") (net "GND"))
 (segment (start 137.16 96.52) (end 137.16 90.17) (width 0.5) (layer "F.Cu") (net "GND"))
 (segment (start 116.84 116.84) (end 118.87 116.84) (width 0.5) (layer "F.Cu") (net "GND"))
 (segment (start 114.11 96.52) (end 114.11 110.87) (width 0.5) (layer "F.Cu") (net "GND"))
 (segment (start 140.81 111.88) (end 137.78 111.88) (width 0.5) (layer "F.Cu") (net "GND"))
 (segment (start 129.6525 82.41) (end 126.6525 85.41) (width 0.5) (layer "F.Cu") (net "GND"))
 (segment (start 123.19 75.853) (end 129.193 75.853) (width 0.5) (layer "F.Cu") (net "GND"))
 (segment (start 136.755 96.925) (end 137.16 96.52) (width 0.5) (layer "F.Cu") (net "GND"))
 (segment (start 131.68 111.89) (end 127.75 107.96) (width 0.5) (layer "F.Cu") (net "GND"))
 (segment (start 120.779 75.848) (end 120.784 75.853) (width 0.5) (layer "F.Cu") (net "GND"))
 (segment (start 115.36 115.36) (end 116.84 116.84) (width 0.5) (layer "F.Cu") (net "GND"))
 (segment (start 110.744 75.848) (end 120.779 75.848) (width 0.5) (layer "F.Cu") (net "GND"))
 (segment (start 137.16 90.17) (end 136.415 89.425) (width 0.5) (layer "F.Cu") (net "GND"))
 (segment (start 131.157 75.853) (end 135.89 71.12) (width 0.5) (layer "F.Cu") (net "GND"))
 (segment (start 129.6525 76.3125) (end 129.6525 82.41) (width 0.5) (layer "F.Cu") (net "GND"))
 (segment (start 115.36 112.12) (end 115.36 115.36) (width 0.5) (layer "F.Cu") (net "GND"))
 (segment (start 101.37 110.87) (end 114.11 110.87) (width 0.5) (layer "F.Cu") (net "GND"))
 (segment (start 100.12 112.12) (end 101.37 110.87) (width 0.5) (layer "F.Cu") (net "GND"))
 (segment (start 100.33 96.52) (end 114.11 96.52) (width 0.5) (layer "F.Cu") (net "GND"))
 (segment (start 129.193 75.853) (end 129.6525 76.3125) (width 0.5) (layer "F.Cu") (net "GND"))
 (segment (start 135.89 68.58) (end 120.6 68.58) (width 0.5) (layer "F.Cu") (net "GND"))
 (segment (start 134.71 89.425) (end 129.6525 84.3675) (width 0.5) (layer "F.Cu") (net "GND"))
 (segment (start 132.71 112.92) (end 132.71 118.95) (width 0.5) (layer "F.Cu") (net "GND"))
 (segment (start 137.77 111.89) (end 131.68 111.89) (width 0.5) (layer "F.Cu") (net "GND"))
 (segment (start 118.49 70.69) (end 115.95 70.69) (width 0.5) (layer "F.Cu") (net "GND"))
 (segment (start 110.28 112.12) (end 110.28 115.71) (width 0.5) (layer "F.Cu") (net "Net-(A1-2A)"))
 (segment (start 110.28 115.71) (end 110.34 115.77) (width 0.5) (layer "F.Cu") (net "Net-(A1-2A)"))
 (segment (start 96.52 74.93) (end 96.52 101.6) (width 0.5) (layer "F.Cu") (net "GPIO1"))
 (segment (start 105.79 70.69) (end 105.79 74.55) (width 0.5) (layer "F.Cu") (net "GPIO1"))
 (segment (start 105.41 74.93) (end 96.52 74.93) (width 0.5) (layer "F.Cu") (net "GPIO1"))
 (segment (start 100.48 101.6) (end 102.66 99.42) (width 0.5) (layer "F.Cu") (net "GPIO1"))
 (segment (start 96.52 101.6) (end 100.48 101.6) (width 0.5) (layer "F.Cu") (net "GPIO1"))
 (segment (start 105.79 74.55) (end 105.41 74.93) (width 0.5) (layer "F.Cu") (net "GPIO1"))
 (segment (start 116.71 98.23) (end 116.71 80.44) (width 0.5) (layer "F.Cu") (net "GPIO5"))
 (segment (start 117.9 99.42) (end 116.71 98.23) (width 0.5) (layer "F.Cu") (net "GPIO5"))
 (segment (start 116.71 80.44) (end 117.96 79.19) (width 0.5) (layer "F.Cu") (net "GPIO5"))
 (segment (start 105.2 99.42) (end 107.74 99.42) (width 0.5) (layer "F.Cu") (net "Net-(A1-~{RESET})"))
 (segment (start 113.41 72.772) (end 113.284 72.898) (width 0.5) (layer "F.Cu") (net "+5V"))
 (segment (start 104.29 90.32) (end 102.72 91.89) (width 0.5) (layer "F.Cu") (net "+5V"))
 (segment (start 109.09 85.52) (end 104.29 90.32) (width 0.5) (layer "F.Cu") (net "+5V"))
 (segment (start 110.744 72.898) (end 113.284 72.898) (width 0.5) (layer "F.Cu") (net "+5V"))
 (segment (start 113.41 70.69) (end 113.41 72.772) (width 0.5) (layer "F.Cu") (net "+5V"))
 (segment (start 110.744 72.898) (end 109.09 74.552) (width 0.5) (layer "F.Cu") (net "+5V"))
 (segment (start 109.09 74.552) (end 109.09 85.52) (width 0.5) (layer "F.Cu") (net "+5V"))
 (segment (start 102.72 91.89) (end 103.02 91.59) (width 0.5) (layer "F.Cu") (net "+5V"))
 (via (at 105.56 89.05) (size 0.6) (drill 0.3) (layers "F.Cu" "B.Cu") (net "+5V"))
 (segment (start 96.52 88.9) (end 96.52 115.57) (width 0.5) (layer "B.Cu") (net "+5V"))
 (segment (start 105.41 88.9) (end 96.52 88.9) (width 0.5) (layer "B.Cu") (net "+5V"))
 (segment (start 99.21 115.57) (end 102.66 112.12) (width 0.5) (layer "B.Cu") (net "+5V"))
 (segment (start 105.56 89.05) (end 105.41 88.9) (width 0.5) (layer "B.Cu") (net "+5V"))
 (segment (start 96.52 115.57) (end 99.21 115.57) (width 0.5) (layer "B.Cu") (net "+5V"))
 (segment (start 112.82 115.71) (end 112.88 115.77) (width 0.5) (layer "F.Cu") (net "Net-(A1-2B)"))
 (segment (start 112.82 112.12) (end 112.82 115.71) (width 0.5) (layer "F.Cu") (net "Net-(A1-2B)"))
 (segment (start 107.74 115.71) (end 107.8 115.77) (width 0.5) (layer "F.Cu") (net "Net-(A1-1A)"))
 (segment (start 107.74 112.12) (end 107.74 115.71) (width 0.5) (layer "F.Cu") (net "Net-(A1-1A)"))
 (segment (start 108.33 70.69) (end 108.33 76.86) (width 0.5) (layer "F.Cu") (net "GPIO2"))
 (segment (start 98.24 99.42) (end 98.24 99.08) (width 0.5) (layer "F.Cu") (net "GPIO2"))
 (segment (start 108.04 77.15) (end 98.13 77.15) (width 0.5) (layer "F.Cu") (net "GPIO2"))
 (segment (start 98.24 99.42) (end 100.12 99.42) (width 0.5) (layer "F.Cu") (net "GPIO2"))
 (segment (start 98.13 77.15) (end 98.13 98.97) (width 0.5) (layer "F.Cu") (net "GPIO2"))
 (segment (start 108.33 76.86) (end 108.04 77.15) (width 0.5) (layer "F.Cu") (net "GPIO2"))
 (segment (start 98.24 99.08) (end 98.13 98.97) (width 0.5) (layer "F.Cu") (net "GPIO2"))
 (segment (start 105.2 112.12) (end 105.2 115.71) (width 0.5) (layer "F.Cu") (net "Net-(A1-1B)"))
 (segment (start 105.2 115.71) (end 105.26 115.77) (width 0.5) (layer "F.Cu") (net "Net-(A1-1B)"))
 (segment (start 120.784 72.903) (end 115.829 72.903) (width 0.5) (layer "F.Cu") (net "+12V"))
 (segment (start 119.83 91.89) (end 120.65 92.71) (width 0.5) (layer "F.Cu") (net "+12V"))
 (segment (start 117.96 91.89) (end 119.83 91.89) (width 0.5) (layer "F.Cu") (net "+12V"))
 (segment (start 120.29 112.12) (end 117.9 112.12) (width 0.5) (layer "F.Cu") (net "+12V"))
 (segment (start 117.96 86.4025) (end 117.96 91.89) (width 0.5) (layer "F.Cu") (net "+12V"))
 (segment (start 120.65 92.71) (end 120.65 111.76) (width 0.5) (layer "F.Cu") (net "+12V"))
 (segment (start 124.9525 79.41) (end 117.96 86.4025) (width 0.5) (layer "F.Cu") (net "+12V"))
 (segment (start 120.65 111.76) (end 120.29 112.12) (width 0.5) (layer "F.Cu") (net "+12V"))
 (segment (start 122.433 72.903) (end 123.19 73.66) (width 0.5) (layer "F.Cu") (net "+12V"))
 (segment (start 115.829 72.903) (end 115.824 72.898) (width 0.2) (layer "F.Cu") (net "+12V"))
 (segment (start 120.784 72.903) (end 122.433 72.903) (width 0.5) (layer "F.Cu") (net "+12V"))
 (via (at 123.19 73.66) (size 0.6) (drill 0.3) (layers "F.Cu" "B.Cu") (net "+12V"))
 (segment (start 124.9525 75.4225) (end 124.9525 79.41) (width 0.5) (layer "B.Cu") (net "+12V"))
 (segment (start 123.19 73.66) (end 124.9525 75.4225) (width 0.5) (layer "B.Cu") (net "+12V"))
 (segment (start 105.26 79.19) (end 107.8 79.19) (width 0.5) (layer "B.Cu") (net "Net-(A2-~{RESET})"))
 (segment (start 105.26 91.89) (end 105.26 94.72) (width 0.5) (layer "F.Cu") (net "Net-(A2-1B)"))
 (segment (start 105.26 94.72) (end 104.94 95.04) (width 0.5) (layer "F.Cu") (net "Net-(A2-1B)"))
 (segment (start 112.88 94.72) (end 112.56 95.04) (width 0.5) (layer "F.Cu") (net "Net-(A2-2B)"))
 (segment (start 112.88 91.89) (end 112.88 94.72) (width 0.5) (layer "F.Cu") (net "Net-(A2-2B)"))
 (segment (start 107.8 91.89) (end 107.8 94.72) (width 0.5) (layer "F.Cu") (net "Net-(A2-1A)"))
 (segment (start 107.8 94.72) (end 107.48 95.04) (width 0.5) (layer "F.Cu") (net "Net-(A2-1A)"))
 (segment (start 110.34 94.72) (end 110.02 95.04) (width 0.5) (layer "F.Cu") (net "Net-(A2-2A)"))
 (segment (start 110.34 91.89) (end 110.34 94.72) (width 0.5) (layer "F.Cu") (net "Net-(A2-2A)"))
 (segment (start 100.71 70.69) (end 100.71 78.66) (width 0.5) (layer "B.Cu") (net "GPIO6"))
 (segment (start 100.71 78.66) (end 100.18 79.19) (width 0.5) (layer "B.Cu") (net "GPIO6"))
 (segment (start 103.25 78.66) (end 102.72 79.19) (width 0.5) (layer "B.Cu") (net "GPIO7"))
 (segment (start 103.25 70.69) (end 103.25 78.66) (width 0.5) (layer "B.Cu") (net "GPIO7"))
 (segment (start 134.71 91.925) (end 134.71 91.985) (width 0.5) (layer "F.Cu") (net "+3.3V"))
 (segment (start 134.71 91.985) (end 123.825 102.87) (width 0.5) (layer "F.Cu") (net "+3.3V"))
 (via (at 123.825 102.87) (size 0.6) (drill 0.3) (layers "F.Cu" "B.Cu") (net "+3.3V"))
 (segment (start 131.14 113.89) (end 137.77 113.89) (width 0.5) (layer "B.Cu") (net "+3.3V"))
 (segment (start 137.77 113.89) (end 140.8 113.89) (width 0.5) (layer "B.Cu") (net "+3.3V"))
 (segment (start 127.75 110.5) (end 123.825 106.575) (width 0.5) (layer "B.Cu") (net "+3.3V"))
 (segment (start 140.8 113.89) (end 140.81 113.88) (width 0.5) (layer "B.Cu") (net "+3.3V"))
 (segment (start 127.75 110.5) (end 131.14 113.89) (width 0.5) (layer "B.Cu") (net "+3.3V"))
 (segment (start 123.825 106.575) (end 123.825 102.87) (width 0.5) (layer "B.Cu") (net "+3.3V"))
 (segment (start 95.63 70.69) (end 99.01 67.31) (width 0.5) (layer "F.Cu") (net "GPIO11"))
 (segment (start 137.795 67.31) (end 138.43 67.945) (width 0.5) (layer "F.Cu") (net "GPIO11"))
 (segment (start 99.01 67.31) (end 137.795 67.31) (width 0.5) (layer "F.Cu") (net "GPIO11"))
 (segment (start 138.43 67.945) (end 138.43 84.455) (width 0.5) (layer "F.Cu") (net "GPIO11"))
 (segment (start 93.75 74.56) (end 93.75 72.57) (width 0.5) (layer "F.Cu") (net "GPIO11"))
 (segment (start 93.75 72.57) (end 95.63 70.69) (width 0.5) (layer "F.Cu") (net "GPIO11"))
 (segment (start 138.4 84.425) (end 134.71 84.425) (width 0.5) (layer "F.Cu") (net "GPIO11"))
 (segment (start 138.43 84.455) (end 138.4 84.425) (width 0.5) (layer "F.Cu") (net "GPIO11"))
 (segment (start 105.41 120.65) (end 144.78 120.65) (width 0.5) (layer "F.Cu") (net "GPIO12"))
 (segment (start 105.84 118.95) (end 105.41 119.38) (width 0.5) (layer "F.Cu") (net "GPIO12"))
 (segment (start 144.78 120.65) (end 144.78 100.965) (width 0.5) (layer "F.Cu") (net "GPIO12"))
 (segment (start 93.75 120.42) (end 93.75 92.32) (width 0.5) (layer "F.Cu") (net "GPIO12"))
 (segment (start 93.98 120.65) (end 93.75 120.42) (width 0.5) (layer "F.Cu") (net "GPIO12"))
 (segment (start 143.165 99.35) (end 134.71 99.35) (width 0.5) (layer "F.Cu") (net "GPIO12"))
 (segment (start 105.79 118.95) (end 105.84 118.95) (width 0.5) (layer "F.Cu") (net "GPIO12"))
 (segment (start 144.78 100.965) (end 143.165 99.35) (width 0.5) (layer "F.Cu") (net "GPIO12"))
 (segment (start 105.41 119.38) (end 105.41 120.65) (width 0.5) (layer "F.Cu") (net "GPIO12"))
 (segment (start 105.41 120.65) (end 93.98 120.65) (width 0.5) (layer "F.Cu") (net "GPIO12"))
 (segment (start 93.75 82.18) (end 93.75 84.7) (width 0.5) (layer "F.Cu") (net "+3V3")))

